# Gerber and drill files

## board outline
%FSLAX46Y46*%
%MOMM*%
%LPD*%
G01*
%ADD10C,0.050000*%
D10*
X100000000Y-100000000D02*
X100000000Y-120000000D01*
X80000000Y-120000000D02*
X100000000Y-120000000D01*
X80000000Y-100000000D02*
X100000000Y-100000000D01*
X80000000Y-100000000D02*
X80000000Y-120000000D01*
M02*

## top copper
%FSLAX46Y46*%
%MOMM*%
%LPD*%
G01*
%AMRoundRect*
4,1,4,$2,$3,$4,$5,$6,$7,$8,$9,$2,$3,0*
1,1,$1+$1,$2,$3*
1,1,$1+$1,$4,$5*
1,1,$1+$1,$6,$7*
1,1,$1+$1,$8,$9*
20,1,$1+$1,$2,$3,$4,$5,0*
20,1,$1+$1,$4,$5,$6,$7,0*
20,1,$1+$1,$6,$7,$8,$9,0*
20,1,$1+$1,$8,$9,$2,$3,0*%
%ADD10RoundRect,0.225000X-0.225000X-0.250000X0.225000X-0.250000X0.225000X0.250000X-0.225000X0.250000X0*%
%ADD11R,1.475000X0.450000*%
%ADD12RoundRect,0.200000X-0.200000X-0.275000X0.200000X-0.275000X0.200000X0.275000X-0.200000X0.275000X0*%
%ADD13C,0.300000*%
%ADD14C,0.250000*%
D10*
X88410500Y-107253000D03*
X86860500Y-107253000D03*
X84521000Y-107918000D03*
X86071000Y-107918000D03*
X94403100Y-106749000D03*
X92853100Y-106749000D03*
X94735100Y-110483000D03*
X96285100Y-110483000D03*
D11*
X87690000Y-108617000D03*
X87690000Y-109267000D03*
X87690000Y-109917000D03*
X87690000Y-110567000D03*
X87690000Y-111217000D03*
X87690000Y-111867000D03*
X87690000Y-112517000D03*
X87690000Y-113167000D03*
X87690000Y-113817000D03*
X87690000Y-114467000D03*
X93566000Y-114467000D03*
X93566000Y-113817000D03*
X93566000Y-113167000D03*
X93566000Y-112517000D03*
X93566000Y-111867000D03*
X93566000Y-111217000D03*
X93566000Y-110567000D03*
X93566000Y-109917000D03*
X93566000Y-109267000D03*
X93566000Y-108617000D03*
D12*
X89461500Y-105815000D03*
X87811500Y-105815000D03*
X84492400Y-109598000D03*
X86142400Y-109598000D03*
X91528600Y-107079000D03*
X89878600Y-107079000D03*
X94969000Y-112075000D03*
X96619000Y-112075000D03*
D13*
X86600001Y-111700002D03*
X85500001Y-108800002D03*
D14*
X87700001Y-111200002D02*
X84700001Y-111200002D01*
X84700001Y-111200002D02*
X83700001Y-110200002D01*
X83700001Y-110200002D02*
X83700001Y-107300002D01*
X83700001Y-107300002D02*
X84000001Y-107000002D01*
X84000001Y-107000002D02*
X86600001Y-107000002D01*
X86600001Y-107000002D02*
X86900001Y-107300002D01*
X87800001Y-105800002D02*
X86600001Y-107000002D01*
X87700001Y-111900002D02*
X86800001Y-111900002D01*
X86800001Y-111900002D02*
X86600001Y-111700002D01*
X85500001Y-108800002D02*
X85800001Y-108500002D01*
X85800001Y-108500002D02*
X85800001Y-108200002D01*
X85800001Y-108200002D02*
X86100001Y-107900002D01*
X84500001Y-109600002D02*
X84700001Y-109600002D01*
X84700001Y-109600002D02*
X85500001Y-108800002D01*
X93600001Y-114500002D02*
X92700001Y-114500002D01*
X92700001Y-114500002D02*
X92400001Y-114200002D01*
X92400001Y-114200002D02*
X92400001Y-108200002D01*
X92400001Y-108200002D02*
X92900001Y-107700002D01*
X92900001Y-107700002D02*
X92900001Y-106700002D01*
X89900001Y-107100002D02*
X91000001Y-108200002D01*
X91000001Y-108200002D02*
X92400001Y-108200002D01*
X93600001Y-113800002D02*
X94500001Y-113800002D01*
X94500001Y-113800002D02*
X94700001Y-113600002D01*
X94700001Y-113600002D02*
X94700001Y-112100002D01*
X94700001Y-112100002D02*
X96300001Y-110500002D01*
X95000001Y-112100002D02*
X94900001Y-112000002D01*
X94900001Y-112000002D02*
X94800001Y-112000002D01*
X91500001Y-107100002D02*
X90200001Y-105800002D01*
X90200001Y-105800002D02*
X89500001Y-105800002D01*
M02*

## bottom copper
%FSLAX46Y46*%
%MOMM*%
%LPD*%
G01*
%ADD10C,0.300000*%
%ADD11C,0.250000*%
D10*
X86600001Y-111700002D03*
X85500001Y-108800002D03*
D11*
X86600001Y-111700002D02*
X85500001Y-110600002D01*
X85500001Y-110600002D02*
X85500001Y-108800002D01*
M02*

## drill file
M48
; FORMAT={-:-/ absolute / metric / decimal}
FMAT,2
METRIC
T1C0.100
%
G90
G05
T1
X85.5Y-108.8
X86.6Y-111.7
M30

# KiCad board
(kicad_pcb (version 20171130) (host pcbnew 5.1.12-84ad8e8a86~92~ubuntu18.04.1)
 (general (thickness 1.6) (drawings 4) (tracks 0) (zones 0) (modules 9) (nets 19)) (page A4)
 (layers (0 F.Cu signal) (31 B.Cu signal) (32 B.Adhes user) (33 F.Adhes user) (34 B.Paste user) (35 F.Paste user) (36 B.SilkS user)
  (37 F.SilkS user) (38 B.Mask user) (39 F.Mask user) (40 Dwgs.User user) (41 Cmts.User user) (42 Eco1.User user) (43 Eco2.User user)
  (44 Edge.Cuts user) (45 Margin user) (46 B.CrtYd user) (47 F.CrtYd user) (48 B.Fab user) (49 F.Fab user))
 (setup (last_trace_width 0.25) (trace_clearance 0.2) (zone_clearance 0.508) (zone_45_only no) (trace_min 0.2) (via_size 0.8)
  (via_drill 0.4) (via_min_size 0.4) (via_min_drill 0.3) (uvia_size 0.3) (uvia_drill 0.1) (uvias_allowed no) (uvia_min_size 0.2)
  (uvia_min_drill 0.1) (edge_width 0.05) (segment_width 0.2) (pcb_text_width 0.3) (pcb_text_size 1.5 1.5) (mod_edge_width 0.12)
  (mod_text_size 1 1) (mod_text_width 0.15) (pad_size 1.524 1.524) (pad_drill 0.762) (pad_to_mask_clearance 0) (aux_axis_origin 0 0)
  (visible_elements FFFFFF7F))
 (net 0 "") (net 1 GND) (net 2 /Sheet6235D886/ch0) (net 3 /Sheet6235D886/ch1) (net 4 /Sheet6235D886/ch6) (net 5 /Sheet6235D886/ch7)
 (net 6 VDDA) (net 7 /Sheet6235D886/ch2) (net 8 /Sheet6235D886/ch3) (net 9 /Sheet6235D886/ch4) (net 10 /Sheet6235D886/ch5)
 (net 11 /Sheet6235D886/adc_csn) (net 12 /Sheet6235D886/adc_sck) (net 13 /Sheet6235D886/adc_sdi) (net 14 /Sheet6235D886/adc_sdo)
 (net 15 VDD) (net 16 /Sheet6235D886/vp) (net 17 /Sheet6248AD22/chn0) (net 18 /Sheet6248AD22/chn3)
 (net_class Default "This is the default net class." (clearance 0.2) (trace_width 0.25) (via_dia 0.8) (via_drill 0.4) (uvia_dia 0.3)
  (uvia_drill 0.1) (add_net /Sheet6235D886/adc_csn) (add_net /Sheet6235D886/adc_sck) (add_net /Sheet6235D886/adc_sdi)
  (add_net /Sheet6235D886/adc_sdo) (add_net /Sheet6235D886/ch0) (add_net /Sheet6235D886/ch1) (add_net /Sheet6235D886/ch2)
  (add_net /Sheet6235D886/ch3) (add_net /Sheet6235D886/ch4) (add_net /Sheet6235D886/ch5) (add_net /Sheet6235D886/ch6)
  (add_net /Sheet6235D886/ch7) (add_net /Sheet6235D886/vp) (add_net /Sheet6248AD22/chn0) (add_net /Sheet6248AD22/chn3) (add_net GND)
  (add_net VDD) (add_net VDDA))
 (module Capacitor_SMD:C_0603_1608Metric (layer F.Cu) (at 87.635500 107.253000)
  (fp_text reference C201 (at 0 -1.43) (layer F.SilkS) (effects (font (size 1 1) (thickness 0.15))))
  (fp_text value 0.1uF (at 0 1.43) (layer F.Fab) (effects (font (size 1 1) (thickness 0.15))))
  (pad 2 smd roundrect (at 0.775 0) (size 0.9 0.95) (layers F.Cu F.Mask F.Paste) (roundrect_rratio 0.25) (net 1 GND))
  (pad 1 smd roundrect (at -0.775 0) (size 0.9 0.95) (layers F.Cu F.Mask F.Paste) (roundrect_rratio 0.25) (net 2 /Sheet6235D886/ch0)))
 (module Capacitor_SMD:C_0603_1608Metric (layer F.Cu) (at 85.296000 107.918000)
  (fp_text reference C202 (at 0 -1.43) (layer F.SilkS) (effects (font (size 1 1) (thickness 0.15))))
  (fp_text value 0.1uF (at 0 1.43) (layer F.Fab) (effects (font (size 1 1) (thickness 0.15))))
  (pad 1 smd roundrect (at -0.775 0) (size 0.9 0.95) (layers F.Cu F.Mask F.Paste) (roundrect_rratio 0.25) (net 1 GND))
  (pad 2 smd roundrect (at 0.775 0) (size 0.9 0.95) (layers F.Cu F.Mask F.Paste) (roundrect_rratio 0.25) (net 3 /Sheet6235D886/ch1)))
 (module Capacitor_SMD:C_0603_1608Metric (layer F.Cu) (at 93.628100 106.749000)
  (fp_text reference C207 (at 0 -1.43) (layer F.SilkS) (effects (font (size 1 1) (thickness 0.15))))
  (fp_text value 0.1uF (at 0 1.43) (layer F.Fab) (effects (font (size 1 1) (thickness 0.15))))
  (pad 2 smd roundrect (at 0.775 0) (size 0.9 0.95) (layers F.Cu F.Mask F.Paste) (roundrect_rratio 0.25) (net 1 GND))
  (pad 1 smd roundrect (at -0.775 0) (size 0.9 0.95) (layers F.Cu F.Mask F.Paste) (roundrect_rratio 0.25) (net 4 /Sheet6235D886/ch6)))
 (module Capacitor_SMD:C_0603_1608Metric (layer F.Cu) (at 95.510100 110.483000)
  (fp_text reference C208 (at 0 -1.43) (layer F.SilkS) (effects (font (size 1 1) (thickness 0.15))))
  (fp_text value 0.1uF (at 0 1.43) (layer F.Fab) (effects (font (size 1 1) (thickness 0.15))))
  (pad 1 smd roundrect (at -0.775 0) (size 0.9 0.95) (layers F.Cu F.Mask F.Paste) (roundrect_rratio 0.25) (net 1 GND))
  (pad 2 smd roundrect (at 0.775 0) (size 0.9 0.95) (layers F.Cu F.Mask F.Paste) (roundrect_rratio 0.25) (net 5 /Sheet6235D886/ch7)))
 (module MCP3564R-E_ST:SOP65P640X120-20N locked (layer F.Cu) (at 90.628000 111.542000)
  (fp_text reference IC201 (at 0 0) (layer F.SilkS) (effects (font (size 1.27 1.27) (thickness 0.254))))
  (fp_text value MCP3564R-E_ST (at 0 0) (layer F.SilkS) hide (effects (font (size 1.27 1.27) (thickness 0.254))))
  (pad 1 smd rect (at -2.938 -2.925 90.000000) (size 0.45 1.475) (layers F.Cu F.Mask F.Paste) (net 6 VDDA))
  (pad 2 smd rect (at -2.938 -2.275 90.000000) (size 0.45 1.475) (layers F.Cu F.Mask F.Paste) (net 1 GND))
  (pad 3 smd rect (at -2.938 -1.625 90.000000) (size 0.45 1.475) (layers F.Cu F.Mask F.Paste) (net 1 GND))
  (pad 4 smd rect (at -2.938 -0.975 90.000000) (size 0.45 1.475) (layers F.Cu F.Mask F.Paste))
  (pad 5 smd rect (at -2.938 -0.325 90.000000) (size 0.45 1.475) (layers F.Cu F.Mask F.Paste) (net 2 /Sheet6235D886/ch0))
  (pad 6 smd rect (at -2.938 0.325 90.000000) (size 0.45 1.475) (layers F.Cu F.Mask F.Paste) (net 3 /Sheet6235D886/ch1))
  (pad 7 smd rect (at -2.938 0.975 90.000000) (size 0.45 1.475) (layers F.Cu F.Mask F.Paste) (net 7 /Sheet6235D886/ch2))
  (pad 8 smd rect (at -2.938 1.625 90.000000) (size 0.45 1.475) (layers F.Cu F.Mask F.Paste) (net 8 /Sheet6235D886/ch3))
  (pad 9 smd rect (at -2.938 2.275 90.000000) (size 0.45 1.475) (layers F.Cu F.Mask F.Paste) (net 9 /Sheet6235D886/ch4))
  (pad 10 smd rect (at -2.938 2.925 90.000000) (size 0.45 1.475) (layers F.Cu F.Mask F.Paste) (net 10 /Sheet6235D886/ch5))
  (pad 11 smd rect (at 2.938 2.925 90.000000) (size 0.45 1.475) (layers F.Cu F.Mask F.Paste) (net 4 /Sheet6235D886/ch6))
  (pad 12 smd rect (at 2.938 2.275 90.000000) (size 0.45 1.475) (layers F.Cu F.Mask F.Paste) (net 5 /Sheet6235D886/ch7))
  (pad 13 smd rect (at 2.938 1.625 90.000000) (size 0.45 1.475) (layers F.Cu F.Mask F.Paste) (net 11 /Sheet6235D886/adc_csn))
  (pad 14 smd rect (at 2.938 0.975 90.000000) (size 0.45 1.475) (layers F.Cu F.Mask F.Paste) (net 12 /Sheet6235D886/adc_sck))
  (pad 15 smd rect (at 2.938 0.325 90.000000) (size 0.45 1.475) (layers F.Cu F.Mask F.Paste) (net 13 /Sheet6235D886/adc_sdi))
  (pad 16 smd rect (at 2.938 -0.325 90.000000) (size 0.45 1.475) (layers F.Cu F.Mask F.Paste) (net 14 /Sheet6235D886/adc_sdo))
  (pad 17 smd rect (at 2.938 -0.975 90.000000) (size 0.45 1.475) (layers F.Cu F.Mask F.Paste))
  (pad 18 smd rect (at 2.938 -1.625 90.000000) (size 0.45 1.475) (layers F.Cu F.Mask F.Paste))
  (pad 19 smd rect (at 2.938 -2.275 90.000000) (size 0.45 1.475) (layers F.Cu F.Mask F.Paste) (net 1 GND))
  (pad 20 smd rect (at 2.938 -2.925 90.000000) (size 0.45 1.475) (layers F.Cu F.Mask F.Paste) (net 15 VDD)))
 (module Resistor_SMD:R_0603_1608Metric (layer F.Cu) (at 88.636500 105.815000)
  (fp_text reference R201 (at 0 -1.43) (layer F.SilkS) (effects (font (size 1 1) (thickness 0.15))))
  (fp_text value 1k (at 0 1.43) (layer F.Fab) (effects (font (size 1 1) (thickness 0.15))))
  (pad 2 smd roundrect (at 0.825 0) (size 0.8 0.95) (layers F.Cu F.Mask F.Paste) (roundrect_rratio 0.25) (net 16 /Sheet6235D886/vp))
  (pad 1 smd roundrect (at -0.825 0) (size 0.8 0.95) (layers F.Cu F.Mask F.Paste) (roundrect_rratio 0.25) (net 2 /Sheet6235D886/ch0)))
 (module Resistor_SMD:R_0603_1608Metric (layer F.Cu) (at 85.317400 109.598000)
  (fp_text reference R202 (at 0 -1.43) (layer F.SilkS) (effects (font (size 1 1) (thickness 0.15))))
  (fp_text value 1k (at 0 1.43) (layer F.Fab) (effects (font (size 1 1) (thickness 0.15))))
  (pad 1 smd roundrect (at -0.825 0) (size 0.8 0.95) (layers F.Cu F.Mask F.Paste) (roundrect_rratio 0.25) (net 3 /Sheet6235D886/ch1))
  (pad 2 smd roundrect (at 0.825 0) (size 0.8 0.95) (layers F.Cu F.Mask F.Paste) (roundrect_rratio 0.25) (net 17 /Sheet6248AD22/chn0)))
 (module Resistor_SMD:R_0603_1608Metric (layer F.Cu) (at 90.703600 107.079000)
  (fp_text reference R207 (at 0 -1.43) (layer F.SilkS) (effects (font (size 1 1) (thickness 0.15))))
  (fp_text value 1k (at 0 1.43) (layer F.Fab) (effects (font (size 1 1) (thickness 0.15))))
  (pad 2 smd roundrect (at 0.825 0) (size 0.8 0.95) (layers F.Cu F.Mask F.Paste) (roundrect_rratio 0.25) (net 16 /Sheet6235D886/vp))
  (pad 1 smd roundrect (at -0.825 0) (size 0.8 0.95) (layers F.Cu F.Mask F.Paste) (roundrect_rratio 0.25) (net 4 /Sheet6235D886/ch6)))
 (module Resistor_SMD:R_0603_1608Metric (layer F.Cu) (at 95.794000 112.075000)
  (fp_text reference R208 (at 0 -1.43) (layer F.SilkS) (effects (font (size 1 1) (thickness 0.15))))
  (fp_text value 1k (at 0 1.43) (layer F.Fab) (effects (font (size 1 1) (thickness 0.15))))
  (pad 1 smd roundrect (at -0.825 0) (size 0.8 0.95) (layers F.Cu F.Mask F.Paste) (roundrect_rratio 0.25) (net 5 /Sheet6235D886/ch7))
  (pad 2 smd roundrect (at 0.825 0) (size 0.8 0.95) (layers F.Cu F.Mask F.Paste) (roundrect_rratio 0.25) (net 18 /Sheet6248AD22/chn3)))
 (gr_line (start 100 100) (end 100 120) (layer Edge.Cuts) (width 0.05))
 (gr_line (start 80 120) (end 100 120) (layer Edge.Cuts) (width 0.05))
 (gr_line (start 80 100) (end 100 100) (layer Edge.Cuts) (width 0.05))
 (gr_line (start 80 100) (end 80 120) (layer Edge.Cuts) (width 0.05))
 (segment (start 87.700001 111.200002) (end 84.700001 111.200002) (width 0.250000) (layer F.Cu) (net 2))
 (segment (start 84.700001 111.200002) (end 83.700001 110.200002) (width 0.250000) (layer F.Cu) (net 2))
 (segment (start 83.700001 110.200002) (end 83.700001 107.300002) (width 0.250000) (layer F.Cu) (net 2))
 (segment (start 83.700001 107.300002) (end 84.000001 107.000002) (width 0.250000) (layer F.Cu) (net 2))
 (segment (start 84.000001 107.000002) (end 86.600001 107.000002) (width 0.250000) (layer F.Cu) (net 2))
 (segment (start 86.600001 107.000002) (end 86.900001 107.300002) (width 0.250000) (layer F.Cu) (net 2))
 (segment (start 87.800001 105.800002) (end 86.600001 107.000002) (width 0.250000) (layer F.Cu) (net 2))
 (segment (start 87.700001 111.900002) (end 86.800001 111.900002) (width 0.250000) (layer F.Cu) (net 3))
 (segment (start 86.800001 111.900002) (end 86.600001 111.700002) (width 0.250000) (layer F.Cu) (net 3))
 (segment (start 86.600001 111.700002) (end 85.500001 110.600002) (width 0.250000) (layer B.Cu) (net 3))
 (segment (start 85.500001 110.600002) (end 85.500001 108.800002) (width 0.250000) (layer B.Cu) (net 3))
 (segment (start 85.500001 108.800002) (end 85.800001 108.500002) (width 0.250000) (layer F.Cu) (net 3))
 (segment (start 85.800001 108.500002) (end 85.800001 108.200002) (width 0.250000) (layer F.Cu) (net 3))
 (segment (start 85.800001 108.200002) (end 86.100001 107.900002) (width 0.250000) (layer F.Cu) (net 3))
 (segment (start 84.500001 109.600002) (end 84.700001 109.600002) (width 0.250000) (layer F.Cu) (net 3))
 (segment (start 84.700001 109.600002) (end 85.500001 108.800002) (width 0.250000) (layer F.Cu) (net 3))
 (via micro (at 86.600001 111.700002) (size 0.300000) (drill 0.100000) (layers F.Cu B.Cu) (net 3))
 (via micro (at 85.500001 108.800002) (size 0.300000) (drill 0.100000) (layers F.Cu B.Cu) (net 3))
 (segment (start 93.600001 114.500002) (end 92.700001 114.500002) (width 0.250000) (layer F.Cu) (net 4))
 (segment (start 92.700001 114.500002) (end 92.400001 114.200002) (width 0.250000) (layer F.Cu) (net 4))
 (segment (start 92.400001 114.200002) (end 92.400001 108.200002) (width 0.250000) (layer F.Cu) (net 4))
 (segment (start 92.400001 108.200002) (end 92.900001 107.700002) (width 0.250000) (layer F.Cu) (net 4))
 (segment (start 92.900001 107.700002) (end 92.900001 106.700002) (width 0.250000) (layer F.Cu) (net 4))
 (segment (start 89.900001 107.100002) (end 91.000001 108.200002) (width 0.250000) (layer F.Cu) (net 4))
 (segment (start 91.000001 108.200002) (end 92.400001 108.200002) (width 0.250000) (layer F.Cu) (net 4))
 (segment (start 93.600001 113.800002) (end 94.500001 113.800002) (width 0.250000) (layer F.Cu) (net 5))
 (segment (start 94.500001 113.800002) (end 94.700001 113.600002) (width 0.250000) (layer F.Cu) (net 5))
 (segment (start 94.700001 113.600002) (end 94.700001 112.100002) (width 0.250000) (layer F.Cu) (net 5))
 (segment (start 94.700001 112.100002) (end 96.300001 110.500002) (width 0.250000) (layer F.Cu) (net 5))
 (segment (start 95.000001 112.100002) (end 94.900001 112.000002) (width 0.250000) (layer F.Cu) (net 5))
 (segment (start 94.900001 112.000002) (end 94.800001 112.000002) (width 0.250000) (layer F.Cu) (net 5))
 (segment (start 91.500001 107.100002) (end 90.200001 105.800002) (width 0.250000) (layer F.Cu) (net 16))
 (segment (start 90.200001 105.800002) (end 89.500001 105.800002) (width 0.250000) (layer F.Cu) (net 16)))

